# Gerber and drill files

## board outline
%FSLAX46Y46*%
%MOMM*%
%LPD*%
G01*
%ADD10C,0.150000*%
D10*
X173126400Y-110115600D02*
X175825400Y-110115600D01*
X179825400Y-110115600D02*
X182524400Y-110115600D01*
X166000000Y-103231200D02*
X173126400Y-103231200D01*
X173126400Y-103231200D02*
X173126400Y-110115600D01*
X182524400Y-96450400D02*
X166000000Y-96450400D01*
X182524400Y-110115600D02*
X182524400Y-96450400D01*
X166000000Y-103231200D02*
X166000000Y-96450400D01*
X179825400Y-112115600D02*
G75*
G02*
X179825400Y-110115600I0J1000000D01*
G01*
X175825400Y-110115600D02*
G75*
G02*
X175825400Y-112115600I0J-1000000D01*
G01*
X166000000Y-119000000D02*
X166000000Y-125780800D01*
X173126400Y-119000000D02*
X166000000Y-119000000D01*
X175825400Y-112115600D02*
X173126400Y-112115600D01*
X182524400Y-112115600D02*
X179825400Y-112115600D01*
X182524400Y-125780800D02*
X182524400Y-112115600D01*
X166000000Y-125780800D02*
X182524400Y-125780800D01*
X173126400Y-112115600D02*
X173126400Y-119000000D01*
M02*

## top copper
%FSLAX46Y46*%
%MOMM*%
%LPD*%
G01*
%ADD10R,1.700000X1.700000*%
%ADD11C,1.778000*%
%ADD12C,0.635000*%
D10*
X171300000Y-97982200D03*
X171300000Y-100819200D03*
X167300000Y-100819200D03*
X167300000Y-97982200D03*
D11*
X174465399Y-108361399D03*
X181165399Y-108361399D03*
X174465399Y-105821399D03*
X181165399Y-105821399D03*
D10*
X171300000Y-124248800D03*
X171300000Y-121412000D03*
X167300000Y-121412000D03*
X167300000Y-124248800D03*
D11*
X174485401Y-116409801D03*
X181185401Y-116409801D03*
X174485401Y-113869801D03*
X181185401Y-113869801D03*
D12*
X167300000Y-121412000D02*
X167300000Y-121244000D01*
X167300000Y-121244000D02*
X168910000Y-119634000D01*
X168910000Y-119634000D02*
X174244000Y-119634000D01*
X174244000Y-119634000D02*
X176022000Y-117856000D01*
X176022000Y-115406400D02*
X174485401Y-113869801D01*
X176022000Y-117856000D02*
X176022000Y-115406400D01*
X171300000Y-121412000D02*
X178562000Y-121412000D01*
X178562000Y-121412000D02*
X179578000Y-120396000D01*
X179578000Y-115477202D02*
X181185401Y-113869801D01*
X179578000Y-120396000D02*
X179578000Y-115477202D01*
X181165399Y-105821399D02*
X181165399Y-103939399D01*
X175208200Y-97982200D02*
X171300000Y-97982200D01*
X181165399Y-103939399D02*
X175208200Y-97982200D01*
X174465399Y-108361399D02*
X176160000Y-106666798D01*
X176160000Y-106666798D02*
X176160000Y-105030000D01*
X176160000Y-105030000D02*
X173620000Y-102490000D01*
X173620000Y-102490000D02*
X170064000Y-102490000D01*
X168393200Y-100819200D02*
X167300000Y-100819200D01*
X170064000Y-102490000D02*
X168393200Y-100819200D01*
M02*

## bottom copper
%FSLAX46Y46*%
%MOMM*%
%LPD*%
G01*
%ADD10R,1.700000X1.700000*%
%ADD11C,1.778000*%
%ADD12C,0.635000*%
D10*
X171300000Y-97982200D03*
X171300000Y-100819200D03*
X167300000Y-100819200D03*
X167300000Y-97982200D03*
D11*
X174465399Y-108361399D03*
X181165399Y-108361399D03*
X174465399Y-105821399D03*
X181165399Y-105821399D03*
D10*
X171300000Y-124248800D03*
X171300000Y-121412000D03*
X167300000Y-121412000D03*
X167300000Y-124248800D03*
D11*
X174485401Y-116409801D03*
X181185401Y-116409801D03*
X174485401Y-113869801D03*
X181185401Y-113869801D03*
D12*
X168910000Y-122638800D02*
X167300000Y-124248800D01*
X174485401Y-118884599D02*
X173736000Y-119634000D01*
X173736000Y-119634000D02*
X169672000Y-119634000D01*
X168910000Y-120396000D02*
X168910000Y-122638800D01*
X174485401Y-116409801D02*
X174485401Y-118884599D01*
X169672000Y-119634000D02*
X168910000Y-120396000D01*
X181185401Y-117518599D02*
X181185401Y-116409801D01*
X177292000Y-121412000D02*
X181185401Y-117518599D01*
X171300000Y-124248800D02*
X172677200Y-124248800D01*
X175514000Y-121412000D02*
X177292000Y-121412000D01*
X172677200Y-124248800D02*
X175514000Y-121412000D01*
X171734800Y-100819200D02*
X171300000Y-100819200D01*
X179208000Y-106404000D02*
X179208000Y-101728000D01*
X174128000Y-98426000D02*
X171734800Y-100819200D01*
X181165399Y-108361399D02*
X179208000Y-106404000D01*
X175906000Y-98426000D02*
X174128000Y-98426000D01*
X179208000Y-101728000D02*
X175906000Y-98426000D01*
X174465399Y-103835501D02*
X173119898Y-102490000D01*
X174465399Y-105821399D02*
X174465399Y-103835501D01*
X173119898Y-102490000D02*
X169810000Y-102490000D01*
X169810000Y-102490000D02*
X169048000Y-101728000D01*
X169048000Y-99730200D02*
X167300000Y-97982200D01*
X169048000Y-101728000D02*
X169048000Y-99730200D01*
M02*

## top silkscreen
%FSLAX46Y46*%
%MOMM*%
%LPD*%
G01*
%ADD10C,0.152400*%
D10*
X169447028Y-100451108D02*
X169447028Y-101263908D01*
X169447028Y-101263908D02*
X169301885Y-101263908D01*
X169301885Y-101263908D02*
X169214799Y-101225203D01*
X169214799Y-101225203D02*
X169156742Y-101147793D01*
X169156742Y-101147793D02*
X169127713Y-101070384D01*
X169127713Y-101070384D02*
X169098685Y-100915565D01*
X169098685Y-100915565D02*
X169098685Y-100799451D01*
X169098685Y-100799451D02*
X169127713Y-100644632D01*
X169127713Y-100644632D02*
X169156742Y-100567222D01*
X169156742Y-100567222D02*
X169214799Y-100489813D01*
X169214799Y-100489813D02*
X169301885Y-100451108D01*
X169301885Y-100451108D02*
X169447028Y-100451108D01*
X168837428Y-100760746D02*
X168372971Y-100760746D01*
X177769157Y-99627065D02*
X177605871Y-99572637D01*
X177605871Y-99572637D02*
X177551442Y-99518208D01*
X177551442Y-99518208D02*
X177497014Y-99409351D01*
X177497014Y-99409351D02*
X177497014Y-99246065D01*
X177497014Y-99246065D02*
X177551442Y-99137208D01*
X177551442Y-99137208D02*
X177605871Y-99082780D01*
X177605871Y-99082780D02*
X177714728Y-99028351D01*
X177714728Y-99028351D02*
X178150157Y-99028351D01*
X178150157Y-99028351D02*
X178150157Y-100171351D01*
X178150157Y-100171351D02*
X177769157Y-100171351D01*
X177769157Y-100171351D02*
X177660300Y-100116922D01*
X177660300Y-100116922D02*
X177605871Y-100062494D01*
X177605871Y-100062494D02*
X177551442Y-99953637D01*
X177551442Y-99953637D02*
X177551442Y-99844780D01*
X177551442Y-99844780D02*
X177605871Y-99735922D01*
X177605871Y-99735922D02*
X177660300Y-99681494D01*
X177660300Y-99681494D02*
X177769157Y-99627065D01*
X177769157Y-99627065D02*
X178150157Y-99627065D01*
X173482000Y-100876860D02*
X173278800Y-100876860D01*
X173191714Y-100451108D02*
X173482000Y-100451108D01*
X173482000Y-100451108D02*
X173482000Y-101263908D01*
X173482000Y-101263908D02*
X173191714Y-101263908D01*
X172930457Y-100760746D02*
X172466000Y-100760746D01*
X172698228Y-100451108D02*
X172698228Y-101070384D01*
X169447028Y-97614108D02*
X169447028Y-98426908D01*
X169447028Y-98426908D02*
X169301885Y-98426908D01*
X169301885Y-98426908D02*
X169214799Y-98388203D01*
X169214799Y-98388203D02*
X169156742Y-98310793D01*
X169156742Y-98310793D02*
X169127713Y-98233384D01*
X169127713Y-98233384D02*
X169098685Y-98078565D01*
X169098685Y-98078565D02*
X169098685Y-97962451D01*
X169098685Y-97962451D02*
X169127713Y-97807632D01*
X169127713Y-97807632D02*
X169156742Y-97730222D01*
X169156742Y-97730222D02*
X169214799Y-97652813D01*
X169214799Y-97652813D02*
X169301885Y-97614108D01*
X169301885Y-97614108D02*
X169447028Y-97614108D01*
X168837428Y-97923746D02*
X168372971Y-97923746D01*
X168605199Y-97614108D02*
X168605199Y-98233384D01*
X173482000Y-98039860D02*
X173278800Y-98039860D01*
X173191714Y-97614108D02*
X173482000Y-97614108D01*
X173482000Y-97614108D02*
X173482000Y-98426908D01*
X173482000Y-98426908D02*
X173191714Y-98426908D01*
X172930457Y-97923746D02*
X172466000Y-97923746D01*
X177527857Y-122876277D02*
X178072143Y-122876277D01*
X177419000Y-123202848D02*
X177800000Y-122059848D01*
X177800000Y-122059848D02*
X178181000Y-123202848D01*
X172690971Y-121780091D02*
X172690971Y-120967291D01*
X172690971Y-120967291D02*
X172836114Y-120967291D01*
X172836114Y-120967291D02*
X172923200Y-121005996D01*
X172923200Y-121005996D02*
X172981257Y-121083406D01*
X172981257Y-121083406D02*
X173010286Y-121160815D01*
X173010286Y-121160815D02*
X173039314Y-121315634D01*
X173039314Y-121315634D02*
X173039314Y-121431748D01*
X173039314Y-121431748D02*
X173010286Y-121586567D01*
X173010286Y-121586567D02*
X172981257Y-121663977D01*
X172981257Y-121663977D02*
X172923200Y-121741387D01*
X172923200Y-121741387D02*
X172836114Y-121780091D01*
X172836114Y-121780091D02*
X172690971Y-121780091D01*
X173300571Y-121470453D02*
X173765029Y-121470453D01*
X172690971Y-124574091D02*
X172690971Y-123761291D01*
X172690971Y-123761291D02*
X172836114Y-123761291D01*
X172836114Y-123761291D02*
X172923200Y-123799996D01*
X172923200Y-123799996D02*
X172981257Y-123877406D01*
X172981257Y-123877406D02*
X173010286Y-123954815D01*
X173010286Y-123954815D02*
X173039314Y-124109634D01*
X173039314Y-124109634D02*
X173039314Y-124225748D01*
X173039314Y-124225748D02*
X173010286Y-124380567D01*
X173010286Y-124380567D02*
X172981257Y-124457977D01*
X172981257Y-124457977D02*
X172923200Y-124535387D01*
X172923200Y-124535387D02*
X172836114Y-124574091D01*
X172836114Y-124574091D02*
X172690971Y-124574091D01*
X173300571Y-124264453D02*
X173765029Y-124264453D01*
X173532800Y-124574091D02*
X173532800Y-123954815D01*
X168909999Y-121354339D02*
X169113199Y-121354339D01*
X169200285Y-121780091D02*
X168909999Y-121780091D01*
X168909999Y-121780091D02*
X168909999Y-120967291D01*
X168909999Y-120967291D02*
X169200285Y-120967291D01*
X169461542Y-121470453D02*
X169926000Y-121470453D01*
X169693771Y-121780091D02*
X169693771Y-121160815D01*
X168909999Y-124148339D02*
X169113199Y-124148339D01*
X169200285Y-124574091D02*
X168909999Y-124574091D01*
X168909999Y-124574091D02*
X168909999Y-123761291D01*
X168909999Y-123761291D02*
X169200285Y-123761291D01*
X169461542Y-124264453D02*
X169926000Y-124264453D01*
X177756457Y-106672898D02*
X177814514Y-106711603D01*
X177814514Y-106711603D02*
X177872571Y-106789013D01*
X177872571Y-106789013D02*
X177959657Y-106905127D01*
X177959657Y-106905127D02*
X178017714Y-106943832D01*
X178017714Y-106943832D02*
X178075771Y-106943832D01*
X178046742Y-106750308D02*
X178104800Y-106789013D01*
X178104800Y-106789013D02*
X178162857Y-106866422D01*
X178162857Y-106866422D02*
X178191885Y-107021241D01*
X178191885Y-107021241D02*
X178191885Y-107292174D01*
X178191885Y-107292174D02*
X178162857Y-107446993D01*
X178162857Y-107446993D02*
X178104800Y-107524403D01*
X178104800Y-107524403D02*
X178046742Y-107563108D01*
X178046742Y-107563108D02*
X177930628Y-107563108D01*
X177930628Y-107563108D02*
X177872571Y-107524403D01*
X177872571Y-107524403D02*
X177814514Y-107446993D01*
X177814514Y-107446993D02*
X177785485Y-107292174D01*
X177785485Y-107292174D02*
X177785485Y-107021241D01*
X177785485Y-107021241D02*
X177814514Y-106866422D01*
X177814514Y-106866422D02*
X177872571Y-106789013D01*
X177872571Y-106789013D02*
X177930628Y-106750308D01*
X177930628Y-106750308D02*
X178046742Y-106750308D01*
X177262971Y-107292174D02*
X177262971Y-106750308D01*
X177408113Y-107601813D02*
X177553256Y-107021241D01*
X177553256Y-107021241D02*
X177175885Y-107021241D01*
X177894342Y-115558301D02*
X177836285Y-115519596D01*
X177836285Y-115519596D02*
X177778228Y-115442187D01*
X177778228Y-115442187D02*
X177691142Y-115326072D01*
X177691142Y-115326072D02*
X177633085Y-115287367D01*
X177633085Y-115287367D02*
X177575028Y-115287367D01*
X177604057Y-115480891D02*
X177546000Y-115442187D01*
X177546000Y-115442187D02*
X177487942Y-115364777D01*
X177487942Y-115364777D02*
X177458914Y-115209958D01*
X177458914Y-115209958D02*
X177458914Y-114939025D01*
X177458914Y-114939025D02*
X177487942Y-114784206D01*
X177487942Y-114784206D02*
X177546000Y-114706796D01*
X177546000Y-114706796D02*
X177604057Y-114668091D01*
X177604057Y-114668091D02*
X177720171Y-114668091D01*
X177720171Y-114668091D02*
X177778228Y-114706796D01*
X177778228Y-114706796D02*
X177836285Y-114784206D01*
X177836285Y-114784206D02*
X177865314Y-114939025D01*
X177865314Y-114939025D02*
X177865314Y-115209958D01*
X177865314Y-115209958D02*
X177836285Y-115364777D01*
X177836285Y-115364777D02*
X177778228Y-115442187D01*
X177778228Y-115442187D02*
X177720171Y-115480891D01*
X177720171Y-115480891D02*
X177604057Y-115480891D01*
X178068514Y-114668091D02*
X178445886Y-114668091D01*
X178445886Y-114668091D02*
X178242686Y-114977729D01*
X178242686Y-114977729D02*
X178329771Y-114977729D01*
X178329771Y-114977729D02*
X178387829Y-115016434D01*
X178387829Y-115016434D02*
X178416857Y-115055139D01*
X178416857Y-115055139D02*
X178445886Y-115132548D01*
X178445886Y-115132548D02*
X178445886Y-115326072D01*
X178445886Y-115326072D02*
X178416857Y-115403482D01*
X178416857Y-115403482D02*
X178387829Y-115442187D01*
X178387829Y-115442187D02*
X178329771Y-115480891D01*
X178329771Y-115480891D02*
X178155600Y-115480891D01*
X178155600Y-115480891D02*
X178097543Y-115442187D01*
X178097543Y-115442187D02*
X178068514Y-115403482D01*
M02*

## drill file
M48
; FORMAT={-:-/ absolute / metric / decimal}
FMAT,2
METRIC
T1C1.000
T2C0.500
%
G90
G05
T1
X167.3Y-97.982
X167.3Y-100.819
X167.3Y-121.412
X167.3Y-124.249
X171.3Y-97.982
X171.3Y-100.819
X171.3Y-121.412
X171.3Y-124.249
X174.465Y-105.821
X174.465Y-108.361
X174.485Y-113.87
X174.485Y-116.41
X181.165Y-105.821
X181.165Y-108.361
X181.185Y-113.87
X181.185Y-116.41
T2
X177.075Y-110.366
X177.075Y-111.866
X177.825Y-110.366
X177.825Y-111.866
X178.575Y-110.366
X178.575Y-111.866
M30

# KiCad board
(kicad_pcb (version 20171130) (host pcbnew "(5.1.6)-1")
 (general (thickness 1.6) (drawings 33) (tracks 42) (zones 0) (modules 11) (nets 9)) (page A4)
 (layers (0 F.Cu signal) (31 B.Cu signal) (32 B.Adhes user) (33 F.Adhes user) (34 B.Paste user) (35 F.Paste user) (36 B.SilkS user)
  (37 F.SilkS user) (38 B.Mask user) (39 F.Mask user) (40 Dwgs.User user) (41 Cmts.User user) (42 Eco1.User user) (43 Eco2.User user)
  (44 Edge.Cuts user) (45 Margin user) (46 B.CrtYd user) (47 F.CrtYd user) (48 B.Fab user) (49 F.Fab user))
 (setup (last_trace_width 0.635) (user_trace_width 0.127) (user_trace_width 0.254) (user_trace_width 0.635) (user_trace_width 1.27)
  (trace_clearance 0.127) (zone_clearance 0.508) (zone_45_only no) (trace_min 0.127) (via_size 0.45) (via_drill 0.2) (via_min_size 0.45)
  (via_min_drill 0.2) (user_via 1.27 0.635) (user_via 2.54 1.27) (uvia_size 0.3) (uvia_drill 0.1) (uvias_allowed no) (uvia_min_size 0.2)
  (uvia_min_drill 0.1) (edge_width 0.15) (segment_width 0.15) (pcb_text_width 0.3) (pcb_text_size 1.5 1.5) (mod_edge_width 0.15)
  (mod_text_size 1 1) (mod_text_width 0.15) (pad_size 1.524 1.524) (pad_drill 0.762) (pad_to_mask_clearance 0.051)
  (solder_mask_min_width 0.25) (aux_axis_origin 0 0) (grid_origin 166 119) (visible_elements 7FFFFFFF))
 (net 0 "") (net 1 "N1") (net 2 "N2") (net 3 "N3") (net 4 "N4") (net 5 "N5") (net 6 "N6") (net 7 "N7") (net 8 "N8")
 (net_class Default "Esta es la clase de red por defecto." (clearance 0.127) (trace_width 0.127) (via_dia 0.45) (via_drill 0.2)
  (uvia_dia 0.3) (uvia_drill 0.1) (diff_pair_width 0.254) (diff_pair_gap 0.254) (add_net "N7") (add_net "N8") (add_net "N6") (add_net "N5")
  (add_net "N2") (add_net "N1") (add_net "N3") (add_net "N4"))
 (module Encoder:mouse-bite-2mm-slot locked (layer F.Cu) (at 177.8254 111.1156)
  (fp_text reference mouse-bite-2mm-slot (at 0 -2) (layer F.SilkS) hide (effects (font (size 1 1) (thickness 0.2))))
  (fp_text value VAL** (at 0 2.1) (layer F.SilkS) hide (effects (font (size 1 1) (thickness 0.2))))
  (pad "" np_thru_hole circle (at 0.75 0.75) (size 0.5 0.5) (drill 0.5) (layers *.Cu *.Mask))
  (pad "" np_thru_hole circle (at -0.75 0.75) (size 0.5 0.5) (drill 0.5) (layers *.Cu *.Mask))
  (pad "" np_thru_hole circle (at -0.75 -0.75) (size 0.5 0.5) (drill 0.5) (layers *.Cu *.Mask))
  (pad "" np_thru_hole circle (at 0.75 -0.75) (size 0.5 0.5) (drill 0.5) (layers *.Cu *.Mask))
  (pad "" np_thru_hole circle (at 0 0.75) (size 0.5 0.5) (drill 0.5) (layers *.Cu *.Mask))
  (pad "" np_thru_hole circle (at 0 -0.75) (size 0.5 0.5) (drill 0.5) (layers *.Cu *.Mask)))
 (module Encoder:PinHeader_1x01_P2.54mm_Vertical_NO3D (layer F.Cu) (at 171.3 97.9822 180)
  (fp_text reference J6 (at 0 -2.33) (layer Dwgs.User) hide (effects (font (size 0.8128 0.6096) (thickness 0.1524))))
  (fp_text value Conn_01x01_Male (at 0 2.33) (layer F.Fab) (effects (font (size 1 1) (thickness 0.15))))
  (pad 1 thru_hole rect (at 0 0 180) (size 1.7 1.7) (drill 1) (layers *.Cu *.Mask) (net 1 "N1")))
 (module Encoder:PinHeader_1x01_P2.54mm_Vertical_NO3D (layer F.Cu) (at 171.3 100.8192 180)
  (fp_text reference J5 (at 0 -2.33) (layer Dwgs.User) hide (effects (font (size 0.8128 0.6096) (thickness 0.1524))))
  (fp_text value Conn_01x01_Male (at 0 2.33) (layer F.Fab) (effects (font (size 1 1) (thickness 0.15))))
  (pad 1 thru_hole rect (at 0 0 180) (size 1.7 1.7) (drill 1) (layers *.Cu *.Mask) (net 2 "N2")))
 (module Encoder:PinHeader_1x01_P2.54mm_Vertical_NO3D (layer F.Cu) (at 167.3 100.8192 180)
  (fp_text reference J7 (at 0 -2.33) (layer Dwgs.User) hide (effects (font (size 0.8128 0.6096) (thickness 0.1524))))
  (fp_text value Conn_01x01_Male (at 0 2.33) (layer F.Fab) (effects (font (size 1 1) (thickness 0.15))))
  (pad 1 thru_hole rect (at 0 0 180) (size 1.7 1.7) (drill 1) (layers *.Cu *.Mask) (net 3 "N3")))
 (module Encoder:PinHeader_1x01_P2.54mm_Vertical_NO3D (layer F.Cu) (at 167.3 97.9822 180)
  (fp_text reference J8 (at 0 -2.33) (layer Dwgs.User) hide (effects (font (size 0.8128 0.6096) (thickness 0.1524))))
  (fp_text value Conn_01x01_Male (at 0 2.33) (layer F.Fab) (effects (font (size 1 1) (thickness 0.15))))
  (pad 1 thru_hole rect (at 0 0 180) (size 1.7 1.7) (drill 1) (layers *.Cu *.Mask) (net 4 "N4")))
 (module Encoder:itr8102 (layer F.Cu) (at 177.815399 107.091399 180)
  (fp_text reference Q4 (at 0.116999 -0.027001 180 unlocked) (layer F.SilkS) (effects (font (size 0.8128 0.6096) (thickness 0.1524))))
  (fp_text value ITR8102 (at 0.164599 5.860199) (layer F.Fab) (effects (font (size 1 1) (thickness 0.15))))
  (pad 4 thru_hole circle (at 3.35 -1.27 180) (size 1.778 1.778) (drill 1) (layers *.Cu *.Mask) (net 3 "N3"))
  (pad 1 thru_hole circle (at -3.35 -1.27 180) (size 1.778 1.778) (drill 1) (layers *.Cu *.Mask) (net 2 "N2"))
  (pad 3 thru_hole circle (at 3.35 1.27 180) (size 1.778 1.778) (drill 1) (layers *.Cu *.Mask) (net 4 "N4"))
  (pad 2 thru_hole circle (at -3.35 1.27 180) (size 1.778 1.778) (drill 1) (layers *.Cu *.Mask) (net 1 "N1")))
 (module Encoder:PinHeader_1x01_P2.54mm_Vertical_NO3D (layer F.Cu) (at 171.3 124.2488)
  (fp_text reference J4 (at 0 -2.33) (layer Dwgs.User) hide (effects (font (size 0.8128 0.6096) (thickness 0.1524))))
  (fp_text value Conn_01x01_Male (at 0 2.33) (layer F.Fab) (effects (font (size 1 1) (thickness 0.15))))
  (pad 1 thru_hole rect (at 0 0) (size 1.7 1.7) (drill 1) (layers *.Cu *.Mask) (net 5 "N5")))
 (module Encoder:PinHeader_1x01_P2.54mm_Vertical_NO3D (layer F.Cu) (at 171.3 121.412)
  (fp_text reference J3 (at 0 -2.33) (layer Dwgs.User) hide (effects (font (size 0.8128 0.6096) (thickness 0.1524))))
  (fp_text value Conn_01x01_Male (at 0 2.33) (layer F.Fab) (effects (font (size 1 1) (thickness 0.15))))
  (pad 1 thru_hole rect (at 0 0) (size 1.7 1.7) (drill 1) (layers *.Cu *.Mask) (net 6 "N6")))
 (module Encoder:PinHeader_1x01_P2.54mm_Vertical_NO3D (layer F.Cu) (at 167.3 121.412)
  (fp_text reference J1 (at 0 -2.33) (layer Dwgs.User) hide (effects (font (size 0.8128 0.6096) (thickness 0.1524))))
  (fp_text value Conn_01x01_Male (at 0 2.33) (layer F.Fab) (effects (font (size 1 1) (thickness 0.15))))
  (pad 1 thru_hole rect (at 0 0) (size 1.7 1.7) (drill 1) (layers *.Cu *.Mask) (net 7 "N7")))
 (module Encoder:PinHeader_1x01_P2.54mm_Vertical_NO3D (layer F.Cu) (at 167.3 124.2488)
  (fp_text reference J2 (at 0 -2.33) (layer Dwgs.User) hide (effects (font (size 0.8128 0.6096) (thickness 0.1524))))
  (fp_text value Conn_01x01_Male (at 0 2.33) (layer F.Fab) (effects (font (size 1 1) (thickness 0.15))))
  (pad 1 thru_hole rect (at 0 0) (size 1.7 1.7) (drill 1) (layers *.Cu *.Mask) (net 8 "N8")))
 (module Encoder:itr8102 (layer F.Cu) (at 177.835401 115.139801)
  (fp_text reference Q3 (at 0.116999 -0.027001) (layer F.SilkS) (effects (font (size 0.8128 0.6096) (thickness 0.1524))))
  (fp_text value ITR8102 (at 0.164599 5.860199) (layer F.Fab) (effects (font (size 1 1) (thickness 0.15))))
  (pad 2 thru_hole circle (at -3.35 1.27) (size 1.778 1.778) (drill 1) (layers *.Cu *.Mask) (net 8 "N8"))
  (pad 3 thru_hole circle (at 3.35 1.27) (size 1.778 1.778) (drill 1) (layers *.Cu *.Mask) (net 5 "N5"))
  (pad 1 thru_hole circle (at -3.35 -1.27) (size 1.778 1.778) (drill 1) (layers *.Cu *.Mask) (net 7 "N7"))
  (pad 4 thru_hole circle (at 3.35 -1.27) (size 1.778 1.778) (drill 1) (layers *.Cu *.Mask) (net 6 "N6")))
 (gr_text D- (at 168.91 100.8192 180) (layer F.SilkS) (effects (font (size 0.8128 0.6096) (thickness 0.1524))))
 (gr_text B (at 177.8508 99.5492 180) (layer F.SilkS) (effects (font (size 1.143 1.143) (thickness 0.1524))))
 (gr_line (start 173.1264 110.1156) (end 175.8254 110.1156) (layer Edge.Cuts) (width 0.15))
 (gr_line (start 179.8254 110.1156) (end 182.5244 110.1156) (layer Edge.Cuts) (width 0.15))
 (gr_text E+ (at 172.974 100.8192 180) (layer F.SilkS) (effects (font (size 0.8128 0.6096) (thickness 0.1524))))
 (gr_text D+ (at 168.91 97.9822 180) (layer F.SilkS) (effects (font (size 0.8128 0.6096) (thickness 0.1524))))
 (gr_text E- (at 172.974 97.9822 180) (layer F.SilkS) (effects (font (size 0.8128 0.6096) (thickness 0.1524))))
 (gr_line (start 166 103.2312) (end 173.1264 103.2312) (layer Edge.Cuts) (width 0.15))
 (gr_line (start 173.1264 103.2312) (end 173.1264 110.1156) (layer Edge.Cuts) (width 0.15))
 (gr_line (start 182.5244 96.4504) (end 166 96.4504) (layer Edge.Cuts) (width 0.15))
 (gr_line (start 182.5244 110.1156) (end 182.5244 96.4504) (layer Edge.Cuts) (width 0.15))
 (gr_line (start 166 103.2312) (end 166 96.4504) (layer Edge.Cuts) (width 0.15))
 (gr_arc (start 179.8254 111.1156) (end 179.8254 110.1156) (angle -180) (layer Edge.Cuts) (width 0.15))
 (gr_arc (start 175.8254 111.1156) (end 175.8254 112.1156) (angle -180) (layer Edge.Cuts) (width 0.15))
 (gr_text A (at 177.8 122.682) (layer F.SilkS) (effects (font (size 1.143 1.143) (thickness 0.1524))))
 (gr_line (start 166 119) (end 166 125.7808) (layer Edge.Cuts) (width 0.15))
 (gr_line (start 173.1264 119) (end 166 119) (layer Edge.Cuts) (width 0.15))
 (gr_line (start 175.8254 112.1156) (end 173.1264 112.1156) (layer Edge.Cuts) (width 0.15))
 (gr_line (start 182.5244 112.1156) (end 179.8254 112.1156) (layer Edge.Cuts) (width 0.15))
 (gr_line (start 182.5244 125.7808) (end 182.5244 112.1156) (layer Edge.Cuts) (width 0.15))
 (gr_line (start 166 125.7808) (end 182.5244 125.7808) (layer Edge.Cuts) (width 0.15))
 (gr_line (start 173.1264 112.1156) (end 173.1264 119) (layer Edge.Cuts) (width 0.15))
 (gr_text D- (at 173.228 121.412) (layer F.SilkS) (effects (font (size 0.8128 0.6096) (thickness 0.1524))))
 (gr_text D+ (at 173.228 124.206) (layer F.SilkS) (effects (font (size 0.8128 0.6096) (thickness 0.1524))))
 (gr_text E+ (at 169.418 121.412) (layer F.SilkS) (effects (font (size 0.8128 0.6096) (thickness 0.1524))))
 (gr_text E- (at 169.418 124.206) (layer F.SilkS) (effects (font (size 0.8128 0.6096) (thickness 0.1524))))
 (segment (start 167.3 121.412) (end 167.3 121.244) (width 0.635) (layer F.Cu) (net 7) (status 30))
 (segment (start 167.3 121.244) (end 168.91 119.634) (width 0.635) (layer F.Cu) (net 7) (status 10))
 (segment (start 168.91 119.634) (end 174.244 119.634) (width 0.635) (layer F.Cu) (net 7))
 (segment (start 174.244 119.634) (end 176.022 117.856) (width 0.635) (layer F.Cu) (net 7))
 (segment (start 176.022 115.4064) (end 174.485401 113.869801) (width 0.635) (layer F.Cu) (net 7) (status 20))
 (segment (start 176.022 117.856) (end 176.022 115.4064) (width 0.635) (layer F.Cu) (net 7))
 (segment (start 168.91 122.6388) (end 167.3 124.2488) (width 0.635) (layer B.Cu) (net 8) (status 20))
 (segment (start 174.485401 118.884599) (end 173.736 119.634) (width 0.635) (layer B.Cu) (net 8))
 (segment (start 173.736 119.634) (end 169.672 119.634) (width 0.635) (layer B.Cu) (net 8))
 (segment (start 168.91 120.396) (end 168.91 122.6388) (width 0.635) (layer B.Cu) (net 8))
 (segment (start 174.485401 116.409801) (end 174.485401 118.884599) (width 0.635) (layer B.Cu) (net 8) (status 10))
 (segment (start 169.672 119.634) (end 168.91 120.396) (width 0.635) (layer B.Cu) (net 8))
 (segment (start 171.3 121.412) (end 178.562 121.412) (width 0.635) (layer F.Cu) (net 6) (status 10))
 (segment (start 178.562 121.412) (end 179.578 120.396) (width 0.635) (layer F.Cu) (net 6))
 (segment (start 179.578 115.477202) (end 181.185401 113.869801) (width 0.635) (layer F.Cu) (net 6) (status 20))
 (segment (start 179.578 120.396) (end 179.578 115.477202) (width 0.635) (layer F.Cu) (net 6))
 (segment (start 181.185401 117.518599) (end 181.185401 116.409801) (width 0.635) (layer B.Cu) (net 5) (status 20))
 (segment (start 177.292 121.412) (end 181.185401 117.518599) (width 0.635) (layer B.Cu) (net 5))
 (segment (start 171.3 124.2488) (end 172.6772 124.2488) (width 0.635) (layer B.Cu) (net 5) (status 10))
 (segment (start 175.514 121.412) (end 177.292 121.412) (width 0.635) (layer B.Cu) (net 5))
 (segment (start 172.6772 124.2488) (end 175.514 121.412) (width 0.635) (layer B.Cu) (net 5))
 (segment (start 171.7348 100.8192) (end 171.3 100.8192) (width 0.635) (layer B.Cu) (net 2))
 (segment (start 179.208 106.404) (end 179.208 101.728) (width 0.635) (layer B.Cu) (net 2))
 (segment (start 174.128 98.426) (end 171.7348 100.8192) (width 0.635) (layer B.Cu) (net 2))
 (segment (start 181.165399 108.361399) (end 179.208 106.404) (width 0.635) (layer B.Cu) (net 2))
 (segment (start 175.906 98.426) (end 174.128 98.426) (width 0.635) (layer B.Cu) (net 2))
 (segment (start 179.208 101.728) (end 175.906 98.426) (width 0.635) (layer B.Cu) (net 2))
 (segment (start 181.165399 105.821399) (end 181.165399 103.939399) (width 0.635) (layer F.Cu) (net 1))
 (segment (start 175.2082 97.9822) (end 171.3 97.9822) (width 0.635) (layer F.Cu) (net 1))
 (segment (start 181.165399 103.939399) (end 175.2082 97.9822) (width 0.635) (layer F.Cu) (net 1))
 (segment (start 174.465399 108.361399) (end 176.16 106.666798) (width 0.635) (layer F.Cu) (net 3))
 (segment (start 176.16 106.666798) (end 176.16 105.03) (width 0.635) (layer F.Cu) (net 3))
 (segment (start 176.16 105.03) (end 173.62 102.49) (width 0.635) (layer F.Cu) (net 3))
 (segment (start 173.62 102.49) (end 170.064 102.49) (width 0.635) (layer F.Cu) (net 3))
 (segment (start 168.3932 100.8192) (end 167.3 100.8192) (width 0.635) (layer F.Cu) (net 3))
 (segment (start 170.064 102.49) (end 168.3932 100.8192) (width 0.635) (layer F.Cu) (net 3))
 (segment (start 174.465399 103.835501) (end 173.119898 102.49) (width 0.635) (layer B.Cu) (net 4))
 (segment (start 174.465399 105.821399) (end 174.465399 103.835501) (width 0.635) (layer B.Cu) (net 4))
 (segment (start 173.119898 102.49) (end 169.81 102.49) (width 0.635) (layer B.Cu) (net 4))
 (segment (start 169.81 102.49) (end 169.048 101.728) (width 0.635) (layer B.Cu) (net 4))
 (segment (start 169.048 99.7302) (end 167.3 97.9822) (width 0.635) (layer B.Cu) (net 4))
 (segment (start 169.048 101.728) (end 169.048 99.7302) (width 0.635) (layer B.Cu) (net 4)))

